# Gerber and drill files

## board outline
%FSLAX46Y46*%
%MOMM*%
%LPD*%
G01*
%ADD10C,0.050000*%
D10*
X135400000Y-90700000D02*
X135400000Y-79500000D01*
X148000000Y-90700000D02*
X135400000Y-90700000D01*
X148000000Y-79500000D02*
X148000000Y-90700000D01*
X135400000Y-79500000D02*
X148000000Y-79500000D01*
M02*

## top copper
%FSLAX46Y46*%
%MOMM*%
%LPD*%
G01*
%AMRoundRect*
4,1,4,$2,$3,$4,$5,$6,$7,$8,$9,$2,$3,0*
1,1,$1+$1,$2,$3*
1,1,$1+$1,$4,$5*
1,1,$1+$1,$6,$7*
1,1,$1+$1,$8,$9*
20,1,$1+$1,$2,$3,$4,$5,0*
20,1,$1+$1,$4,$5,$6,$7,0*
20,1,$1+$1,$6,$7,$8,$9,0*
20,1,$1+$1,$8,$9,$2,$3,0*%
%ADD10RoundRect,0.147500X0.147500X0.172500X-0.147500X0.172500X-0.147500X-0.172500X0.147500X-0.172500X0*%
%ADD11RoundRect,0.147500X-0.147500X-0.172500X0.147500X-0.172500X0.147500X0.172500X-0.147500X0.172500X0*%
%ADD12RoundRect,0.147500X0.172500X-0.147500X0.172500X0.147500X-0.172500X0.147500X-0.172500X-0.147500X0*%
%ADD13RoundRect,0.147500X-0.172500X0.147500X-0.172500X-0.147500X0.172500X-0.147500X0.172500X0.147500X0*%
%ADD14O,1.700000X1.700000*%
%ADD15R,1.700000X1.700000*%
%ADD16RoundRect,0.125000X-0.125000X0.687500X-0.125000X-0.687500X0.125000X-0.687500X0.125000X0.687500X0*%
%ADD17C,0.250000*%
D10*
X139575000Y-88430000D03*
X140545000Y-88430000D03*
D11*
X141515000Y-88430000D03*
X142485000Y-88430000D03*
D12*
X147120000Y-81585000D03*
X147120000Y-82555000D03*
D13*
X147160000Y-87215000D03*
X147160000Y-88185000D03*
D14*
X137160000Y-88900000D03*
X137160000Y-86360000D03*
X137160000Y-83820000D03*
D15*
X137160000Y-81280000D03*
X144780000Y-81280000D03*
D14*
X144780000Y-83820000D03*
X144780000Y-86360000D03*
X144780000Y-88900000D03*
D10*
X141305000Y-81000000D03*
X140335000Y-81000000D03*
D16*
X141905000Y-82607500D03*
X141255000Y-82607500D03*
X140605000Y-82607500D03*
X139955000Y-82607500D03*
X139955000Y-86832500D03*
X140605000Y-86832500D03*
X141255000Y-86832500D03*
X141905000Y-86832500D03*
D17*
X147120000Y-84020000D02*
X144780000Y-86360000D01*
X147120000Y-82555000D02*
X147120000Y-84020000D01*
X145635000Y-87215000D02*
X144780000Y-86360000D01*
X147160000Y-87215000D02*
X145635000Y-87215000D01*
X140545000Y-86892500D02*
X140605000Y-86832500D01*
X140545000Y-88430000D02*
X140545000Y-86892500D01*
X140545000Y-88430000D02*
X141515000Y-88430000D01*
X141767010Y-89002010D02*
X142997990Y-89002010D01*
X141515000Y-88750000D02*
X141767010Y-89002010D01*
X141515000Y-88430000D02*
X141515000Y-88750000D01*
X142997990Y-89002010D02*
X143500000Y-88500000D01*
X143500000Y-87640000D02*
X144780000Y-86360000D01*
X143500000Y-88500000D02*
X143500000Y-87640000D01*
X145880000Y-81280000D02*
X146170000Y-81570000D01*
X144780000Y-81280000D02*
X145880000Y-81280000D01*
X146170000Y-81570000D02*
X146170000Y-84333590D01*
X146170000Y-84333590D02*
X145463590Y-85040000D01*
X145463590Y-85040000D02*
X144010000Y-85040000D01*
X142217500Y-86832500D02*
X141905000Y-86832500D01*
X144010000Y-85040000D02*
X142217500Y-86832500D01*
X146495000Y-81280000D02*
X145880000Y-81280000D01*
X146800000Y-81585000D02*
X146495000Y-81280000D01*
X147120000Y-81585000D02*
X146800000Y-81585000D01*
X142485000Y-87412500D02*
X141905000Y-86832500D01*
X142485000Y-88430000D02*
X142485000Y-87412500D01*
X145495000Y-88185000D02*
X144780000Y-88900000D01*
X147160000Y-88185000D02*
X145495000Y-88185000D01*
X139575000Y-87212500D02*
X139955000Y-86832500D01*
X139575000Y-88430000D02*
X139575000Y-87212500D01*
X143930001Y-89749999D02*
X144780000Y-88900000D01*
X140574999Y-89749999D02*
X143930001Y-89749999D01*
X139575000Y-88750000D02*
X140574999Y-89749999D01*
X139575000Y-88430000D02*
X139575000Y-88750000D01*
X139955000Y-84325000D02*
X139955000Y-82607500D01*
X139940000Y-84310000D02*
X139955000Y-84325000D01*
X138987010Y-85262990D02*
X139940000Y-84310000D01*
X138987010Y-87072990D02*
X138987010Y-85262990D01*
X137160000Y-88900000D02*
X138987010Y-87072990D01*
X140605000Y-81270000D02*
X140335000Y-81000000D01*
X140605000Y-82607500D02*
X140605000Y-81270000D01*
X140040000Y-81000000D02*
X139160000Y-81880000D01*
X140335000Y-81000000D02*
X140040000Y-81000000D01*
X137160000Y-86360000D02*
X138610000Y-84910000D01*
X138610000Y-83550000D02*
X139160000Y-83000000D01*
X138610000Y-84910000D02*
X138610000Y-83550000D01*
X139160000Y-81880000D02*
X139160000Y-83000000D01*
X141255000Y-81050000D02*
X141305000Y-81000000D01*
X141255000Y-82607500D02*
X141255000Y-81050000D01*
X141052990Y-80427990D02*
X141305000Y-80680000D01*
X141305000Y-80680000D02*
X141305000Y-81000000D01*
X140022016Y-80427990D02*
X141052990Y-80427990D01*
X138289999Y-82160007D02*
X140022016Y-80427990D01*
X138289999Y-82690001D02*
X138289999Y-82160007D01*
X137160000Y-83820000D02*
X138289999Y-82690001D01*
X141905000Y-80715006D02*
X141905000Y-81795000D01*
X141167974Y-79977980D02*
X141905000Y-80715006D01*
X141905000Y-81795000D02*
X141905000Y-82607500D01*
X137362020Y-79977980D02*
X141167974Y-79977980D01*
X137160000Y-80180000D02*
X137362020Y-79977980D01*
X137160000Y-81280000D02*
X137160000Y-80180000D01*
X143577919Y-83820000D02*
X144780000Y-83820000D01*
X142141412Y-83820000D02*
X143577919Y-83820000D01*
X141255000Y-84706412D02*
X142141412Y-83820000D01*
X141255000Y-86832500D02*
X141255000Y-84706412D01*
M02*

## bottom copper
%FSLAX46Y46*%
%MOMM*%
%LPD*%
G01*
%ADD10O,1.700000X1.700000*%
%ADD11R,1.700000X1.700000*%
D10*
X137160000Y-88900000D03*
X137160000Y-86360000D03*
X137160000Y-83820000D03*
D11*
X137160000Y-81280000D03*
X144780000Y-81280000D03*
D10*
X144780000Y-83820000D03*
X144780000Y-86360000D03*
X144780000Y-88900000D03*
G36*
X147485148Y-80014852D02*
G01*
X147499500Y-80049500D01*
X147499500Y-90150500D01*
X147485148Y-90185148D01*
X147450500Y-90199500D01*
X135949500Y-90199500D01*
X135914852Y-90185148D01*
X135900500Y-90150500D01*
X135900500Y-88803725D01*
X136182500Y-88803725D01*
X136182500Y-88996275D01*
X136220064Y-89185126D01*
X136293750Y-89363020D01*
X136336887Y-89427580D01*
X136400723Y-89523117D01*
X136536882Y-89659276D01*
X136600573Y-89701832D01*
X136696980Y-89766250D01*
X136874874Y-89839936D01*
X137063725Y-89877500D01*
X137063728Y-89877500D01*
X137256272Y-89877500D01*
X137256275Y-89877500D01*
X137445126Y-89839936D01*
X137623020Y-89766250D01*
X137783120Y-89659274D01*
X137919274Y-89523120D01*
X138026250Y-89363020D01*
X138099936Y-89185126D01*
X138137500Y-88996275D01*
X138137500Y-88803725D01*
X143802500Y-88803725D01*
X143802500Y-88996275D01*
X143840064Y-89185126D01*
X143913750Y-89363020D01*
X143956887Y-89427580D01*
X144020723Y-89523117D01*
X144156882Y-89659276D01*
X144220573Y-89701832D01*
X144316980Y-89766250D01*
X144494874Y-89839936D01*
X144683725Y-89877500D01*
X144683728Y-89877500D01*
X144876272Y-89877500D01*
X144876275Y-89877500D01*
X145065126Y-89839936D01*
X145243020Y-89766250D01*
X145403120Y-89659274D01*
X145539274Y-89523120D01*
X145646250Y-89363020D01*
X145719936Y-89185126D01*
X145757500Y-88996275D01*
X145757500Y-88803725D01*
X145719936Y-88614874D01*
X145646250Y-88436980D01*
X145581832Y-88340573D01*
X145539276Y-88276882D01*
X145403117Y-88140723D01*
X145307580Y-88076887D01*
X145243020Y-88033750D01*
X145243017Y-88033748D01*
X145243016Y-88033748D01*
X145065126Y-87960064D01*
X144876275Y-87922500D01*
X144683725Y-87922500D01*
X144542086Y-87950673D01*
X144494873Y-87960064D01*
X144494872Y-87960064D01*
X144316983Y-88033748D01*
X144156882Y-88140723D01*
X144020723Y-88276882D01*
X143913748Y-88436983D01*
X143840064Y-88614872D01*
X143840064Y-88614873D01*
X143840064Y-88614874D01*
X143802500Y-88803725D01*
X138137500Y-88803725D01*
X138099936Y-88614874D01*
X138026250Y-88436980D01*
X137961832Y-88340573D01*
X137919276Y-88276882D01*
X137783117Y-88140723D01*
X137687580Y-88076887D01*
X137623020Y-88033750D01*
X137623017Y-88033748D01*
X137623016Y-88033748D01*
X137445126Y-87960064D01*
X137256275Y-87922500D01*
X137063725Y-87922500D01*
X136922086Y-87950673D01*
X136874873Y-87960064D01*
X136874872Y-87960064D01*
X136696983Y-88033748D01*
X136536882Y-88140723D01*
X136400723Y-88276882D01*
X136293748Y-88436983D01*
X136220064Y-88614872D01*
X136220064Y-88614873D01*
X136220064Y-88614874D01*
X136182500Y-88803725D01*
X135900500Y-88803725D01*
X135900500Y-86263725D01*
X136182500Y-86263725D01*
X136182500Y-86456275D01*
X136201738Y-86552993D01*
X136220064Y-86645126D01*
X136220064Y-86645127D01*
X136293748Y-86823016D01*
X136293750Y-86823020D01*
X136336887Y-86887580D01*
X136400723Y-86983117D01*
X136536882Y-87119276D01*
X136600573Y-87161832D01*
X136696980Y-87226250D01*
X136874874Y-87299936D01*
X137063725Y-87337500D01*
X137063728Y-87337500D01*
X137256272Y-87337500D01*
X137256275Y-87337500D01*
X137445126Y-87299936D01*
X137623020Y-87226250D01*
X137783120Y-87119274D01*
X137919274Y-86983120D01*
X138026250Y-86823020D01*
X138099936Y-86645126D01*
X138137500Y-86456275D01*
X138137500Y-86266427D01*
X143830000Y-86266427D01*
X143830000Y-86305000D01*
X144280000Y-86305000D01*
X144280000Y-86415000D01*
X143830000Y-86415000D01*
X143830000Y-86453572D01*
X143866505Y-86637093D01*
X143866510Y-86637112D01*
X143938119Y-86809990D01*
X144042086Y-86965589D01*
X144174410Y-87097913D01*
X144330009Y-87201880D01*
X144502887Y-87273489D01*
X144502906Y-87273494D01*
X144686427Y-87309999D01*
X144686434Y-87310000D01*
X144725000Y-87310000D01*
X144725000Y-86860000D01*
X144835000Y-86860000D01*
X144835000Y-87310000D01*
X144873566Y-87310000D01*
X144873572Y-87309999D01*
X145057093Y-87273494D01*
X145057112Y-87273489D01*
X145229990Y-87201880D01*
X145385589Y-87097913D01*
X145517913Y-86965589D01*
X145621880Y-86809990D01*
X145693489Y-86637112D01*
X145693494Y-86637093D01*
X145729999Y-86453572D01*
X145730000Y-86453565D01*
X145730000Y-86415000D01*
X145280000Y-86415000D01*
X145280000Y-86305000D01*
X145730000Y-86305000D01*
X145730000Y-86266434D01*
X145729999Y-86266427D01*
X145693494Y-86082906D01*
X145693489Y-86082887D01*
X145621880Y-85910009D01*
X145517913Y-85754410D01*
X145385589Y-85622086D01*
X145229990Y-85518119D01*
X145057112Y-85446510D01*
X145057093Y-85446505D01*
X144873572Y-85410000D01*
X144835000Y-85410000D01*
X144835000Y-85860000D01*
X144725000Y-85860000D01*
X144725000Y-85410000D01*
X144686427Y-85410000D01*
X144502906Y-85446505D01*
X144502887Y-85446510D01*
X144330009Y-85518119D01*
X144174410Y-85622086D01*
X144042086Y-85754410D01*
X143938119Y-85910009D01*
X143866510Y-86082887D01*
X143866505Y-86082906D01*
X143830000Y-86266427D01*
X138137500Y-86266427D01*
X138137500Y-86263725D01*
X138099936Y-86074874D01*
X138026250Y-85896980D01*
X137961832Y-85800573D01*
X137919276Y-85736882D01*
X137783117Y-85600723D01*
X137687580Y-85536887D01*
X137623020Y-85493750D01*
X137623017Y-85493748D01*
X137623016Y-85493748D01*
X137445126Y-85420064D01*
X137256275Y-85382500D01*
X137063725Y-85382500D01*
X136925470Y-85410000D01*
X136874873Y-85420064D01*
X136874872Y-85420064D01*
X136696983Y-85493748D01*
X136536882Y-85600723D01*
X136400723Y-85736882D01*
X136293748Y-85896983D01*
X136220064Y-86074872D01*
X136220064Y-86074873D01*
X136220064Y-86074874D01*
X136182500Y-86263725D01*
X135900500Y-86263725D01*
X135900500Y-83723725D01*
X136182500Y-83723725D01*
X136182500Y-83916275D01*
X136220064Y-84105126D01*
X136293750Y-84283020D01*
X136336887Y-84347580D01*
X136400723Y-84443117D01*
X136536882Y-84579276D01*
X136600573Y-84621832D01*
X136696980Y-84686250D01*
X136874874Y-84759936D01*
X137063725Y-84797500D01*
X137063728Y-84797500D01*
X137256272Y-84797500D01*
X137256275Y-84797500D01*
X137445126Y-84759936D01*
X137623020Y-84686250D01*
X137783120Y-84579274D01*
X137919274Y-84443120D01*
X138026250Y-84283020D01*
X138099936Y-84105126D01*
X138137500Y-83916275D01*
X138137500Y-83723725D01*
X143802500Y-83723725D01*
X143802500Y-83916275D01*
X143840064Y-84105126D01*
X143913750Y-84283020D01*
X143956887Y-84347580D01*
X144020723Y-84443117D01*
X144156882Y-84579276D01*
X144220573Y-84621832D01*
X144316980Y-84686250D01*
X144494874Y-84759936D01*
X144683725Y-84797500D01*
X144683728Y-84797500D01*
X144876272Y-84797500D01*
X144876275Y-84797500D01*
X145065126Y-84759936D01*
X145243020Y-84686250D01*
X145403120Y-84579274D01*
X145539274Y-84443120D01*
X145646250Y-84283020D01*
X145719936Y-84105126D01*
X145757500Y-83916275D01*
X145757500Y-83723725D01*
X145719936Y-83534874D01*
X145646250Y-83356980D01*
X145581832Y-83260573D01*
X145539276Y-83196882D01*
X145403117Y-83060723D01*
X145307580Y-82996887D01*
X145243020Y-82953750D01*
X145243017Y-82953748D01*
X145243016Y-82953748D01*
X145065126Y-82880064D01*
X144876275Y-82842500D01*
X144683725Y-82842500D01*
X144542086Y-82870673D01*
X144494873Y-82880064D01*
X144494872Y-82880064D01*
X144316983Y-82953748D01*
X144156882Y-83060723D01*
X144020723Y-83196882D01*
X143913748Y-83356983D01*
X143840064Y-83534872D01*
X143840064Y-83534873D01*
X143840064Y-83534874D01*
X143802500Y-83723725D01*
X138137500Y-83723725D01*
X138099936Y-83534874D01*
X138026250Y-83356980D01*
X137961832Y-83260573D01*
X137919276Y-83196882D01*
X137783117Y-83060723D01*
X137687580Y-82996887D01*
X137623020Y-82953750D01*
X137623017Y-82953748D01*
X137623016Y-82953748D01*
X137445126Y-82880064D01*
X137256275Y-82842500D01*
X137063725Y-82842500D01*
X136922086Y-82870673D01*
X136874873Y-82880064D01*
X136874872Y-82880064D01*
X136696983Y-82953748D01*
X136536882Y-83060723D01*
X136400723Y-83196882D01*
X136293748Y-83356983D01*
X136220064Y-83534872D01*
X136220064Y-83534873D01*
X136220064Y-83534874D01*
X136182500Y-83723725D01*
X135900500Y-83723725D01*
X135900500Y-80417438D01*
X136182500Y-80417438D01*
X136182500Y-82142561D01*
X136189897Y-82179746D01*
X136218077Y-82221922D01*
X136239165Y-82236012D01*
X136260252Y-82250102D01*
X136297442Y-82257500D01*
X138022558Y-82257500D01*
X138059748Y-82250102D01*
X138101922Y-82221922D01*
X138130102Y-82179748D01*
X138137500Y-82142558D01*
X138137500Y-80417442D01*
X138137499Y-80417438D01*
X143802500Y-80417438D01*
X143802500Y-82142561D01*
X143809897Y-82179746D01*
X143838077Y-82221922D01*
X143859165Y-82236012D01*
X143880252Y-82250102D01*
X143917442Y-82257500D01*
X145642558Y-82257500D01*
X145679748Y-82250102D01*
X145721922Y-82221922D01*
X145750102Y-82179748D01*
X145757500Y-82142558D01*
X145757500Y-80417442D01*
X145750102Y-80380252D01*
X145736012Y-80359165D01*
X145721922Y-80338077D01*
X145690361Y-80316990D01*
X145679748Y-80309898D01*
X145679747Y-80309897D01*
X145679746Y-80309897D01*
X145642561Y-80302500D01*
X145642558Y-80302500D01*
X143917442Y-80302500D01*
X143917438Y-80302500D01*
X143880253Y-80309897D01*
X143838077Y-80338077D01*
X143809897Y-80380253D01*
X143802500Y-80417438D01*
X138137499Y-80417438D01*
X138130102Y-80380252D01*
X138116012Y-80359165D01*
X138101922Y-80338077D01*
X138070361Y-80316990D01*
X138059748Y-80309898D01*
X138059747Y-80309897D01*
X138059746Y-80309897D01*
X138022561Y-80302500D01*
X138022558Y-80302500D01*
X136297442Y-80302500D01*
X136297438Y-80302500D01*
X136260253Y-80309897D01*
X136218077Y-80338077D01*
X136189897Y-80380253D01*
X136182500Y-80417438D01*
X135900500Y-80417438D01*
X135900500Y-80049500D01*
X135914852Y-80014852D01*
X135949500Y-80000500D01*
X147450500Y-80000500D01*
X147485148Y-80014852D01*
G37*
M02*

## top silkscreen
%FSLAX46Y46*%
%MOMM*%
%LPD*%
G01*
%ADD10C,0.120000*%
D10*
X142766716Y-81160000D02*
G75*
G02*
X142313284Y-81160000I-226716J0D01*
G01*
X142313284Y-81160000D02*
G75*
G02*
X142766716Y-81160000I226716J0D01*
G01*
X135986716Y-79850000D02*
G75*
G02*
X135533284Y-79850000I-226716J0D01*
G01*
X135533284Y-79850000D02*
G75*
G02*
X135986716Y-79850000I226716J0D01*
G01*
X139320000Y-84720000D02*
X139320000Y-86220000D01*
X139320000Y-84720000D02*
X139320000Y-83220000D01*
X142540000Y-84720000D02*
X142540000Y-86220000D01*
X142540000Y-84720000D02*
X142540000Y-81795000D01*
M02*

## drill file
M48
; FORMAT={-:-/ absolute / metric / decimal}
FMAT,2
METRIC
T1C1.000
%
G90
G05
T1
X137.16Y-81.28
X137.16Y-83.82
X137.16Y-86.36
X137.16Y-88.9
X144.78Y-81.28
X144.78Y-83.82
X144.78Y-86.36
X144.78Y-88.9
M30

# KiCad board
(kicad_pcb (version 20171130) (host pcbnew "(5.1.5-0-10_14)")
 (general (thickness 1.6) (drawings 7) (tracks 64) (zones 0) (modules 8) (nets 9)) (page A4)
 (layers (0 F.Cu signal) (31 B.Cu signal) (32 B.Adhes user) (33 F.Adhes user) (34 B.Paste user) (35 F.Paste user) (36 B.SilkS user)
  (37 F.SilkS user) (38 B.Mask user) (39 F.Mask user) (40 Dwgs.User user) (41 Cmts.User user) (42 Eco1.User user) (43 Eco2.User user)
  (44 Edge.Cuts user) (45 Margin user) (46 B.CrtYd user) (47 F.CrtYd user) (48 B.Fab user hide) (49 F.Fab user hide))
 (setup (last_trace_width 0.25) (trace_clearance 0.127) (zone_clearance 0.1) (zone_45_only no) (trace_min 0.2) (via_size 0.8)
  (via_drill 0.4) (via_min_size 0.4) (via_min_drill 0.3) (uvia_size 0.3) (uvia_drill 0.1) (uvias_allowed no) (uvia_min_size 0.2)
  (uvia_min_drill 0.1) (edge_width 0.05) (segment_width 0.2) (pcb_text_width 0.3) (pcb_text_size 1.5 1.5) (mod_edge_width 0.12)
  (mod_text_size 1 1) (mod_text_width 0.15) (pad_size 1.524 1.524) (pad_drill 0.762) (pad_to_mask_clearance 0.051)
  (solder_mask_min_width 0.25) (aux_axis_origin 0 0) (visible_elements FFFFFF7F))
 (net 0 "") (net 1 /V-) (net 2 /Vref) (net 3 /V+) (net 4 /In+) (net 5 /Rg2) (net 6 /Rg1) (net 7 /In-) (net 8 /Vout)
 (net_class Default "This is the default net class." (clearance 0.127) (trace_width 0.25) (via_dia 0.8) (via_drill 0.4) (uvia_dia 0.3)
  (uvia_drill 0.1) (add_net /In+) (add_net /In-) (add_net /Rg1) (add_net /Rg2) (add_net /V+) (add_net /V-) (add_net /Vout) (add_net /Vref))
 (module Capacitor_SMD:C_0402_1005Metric (layer F.Cu) (at 140.06 88.43 180)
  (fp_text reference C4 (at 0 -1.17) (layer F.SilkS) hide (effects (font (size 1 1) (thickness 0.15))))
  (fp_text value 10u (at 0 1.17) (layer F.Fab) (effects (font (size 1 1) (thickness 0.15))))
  (pad 2 smd roundrect (at 0.485 0 180) (size 0.59 0.64) (layers F.Cu F.Paste F.Mask) (roundrect_rratio 0.25) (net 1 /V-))
  (pad 1 smd roundrect (at -0.485 0 180) (size 0.59 0.64) (layers F.Cu F.Paste F.Mask) (roundrect_rratio 0.25) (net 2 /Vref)))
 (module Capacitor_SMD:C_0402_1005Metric (layer F.Cu) (at 142 88.43)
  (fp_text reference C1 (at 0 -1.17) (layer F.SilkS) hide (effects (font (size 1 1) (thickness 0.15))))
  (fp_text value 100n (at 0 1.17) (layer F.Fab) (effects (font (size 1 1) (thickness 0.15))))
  (pad 1 smd roundrect (at -0.485 0) (size 0.59 0.64) (layers F.Cu F.Paste F.Mask) (roundrect_rratio 0.25) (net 2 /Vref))
  (pad 2 smd roundrect (at 0.485 0) (size 0.59 0.64) (layers F.Cu F.Paste F.Mask) (roundrect_rratio 0.25) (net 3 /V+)))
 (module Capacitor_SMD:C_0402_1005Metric (layer F.Cu) (at 147.12 82.07 90)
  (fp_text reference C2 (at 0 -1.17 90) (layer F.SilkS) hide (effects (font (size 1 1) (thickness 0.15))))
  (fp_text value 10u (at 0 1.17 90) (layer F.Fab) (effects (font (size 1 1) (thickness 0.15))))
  (pad 2 smd roundrect (at 0.485 0 90) (size 0.59 0.64) (layers F.Cu F.Paste F.Mask) (roundrect_rratio 0.25) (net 3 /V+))
  (pad 1 smd roundrect (at -0.485 0 90) (size 0.59 0.64) (layers F.Cu F.Paste F.Mask) (roundrect_rratio 0.25) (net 2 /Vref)))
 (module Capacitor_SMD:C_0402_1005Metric (layer F.Cu) (at 147.16 87.7 270)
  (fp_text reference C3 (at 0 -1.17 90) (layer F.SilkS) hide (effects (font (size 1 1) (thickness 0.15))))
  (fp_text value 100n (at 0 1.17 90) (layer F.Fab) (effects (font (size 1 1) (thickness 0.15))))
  (pad 1 smd roundrect (at -0.485 0 270) (size 0.59 0.64) (layers F.Cu F.Paste F.Mask) (roundrect_rratio 0.25) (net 2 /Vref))
  (pad 2 smd roundrect (at 0.485 0 270) (size 0.59 0.64) (layers F.Cu F.Paste F.Mask) (roundrect_rratio 0.25) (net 1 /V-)))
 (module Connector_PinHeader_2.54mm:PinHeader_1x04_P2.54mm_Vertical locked (layer B.Cu) (at 137.16 81.28 180)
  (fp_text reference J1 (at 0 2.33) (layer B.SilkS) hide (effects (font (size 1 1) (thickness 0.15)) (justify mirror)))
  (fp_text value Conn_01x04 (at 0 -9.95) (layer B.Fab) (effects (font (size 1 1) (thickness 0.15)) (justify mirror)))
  (pad 4 thru_hole oval (at 0 -7.62 180) (size 1.7 1.7) (drill 1) (layers *.Cu *.Mask) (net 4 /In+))
  (pad 3 thru_hole oval (at 0 -5.08 180) (size 1.7 1.7) (drill 1) (layers *.Cu *.Mask) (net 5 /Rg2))
  (pad 2 thru_hole oval (at 0 -2.54 180) (size 1.7 1.7) (drill 1) (layers *.Cu *.Mask) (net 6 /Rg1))
  (pad 1 thru_hole rect (at 0 0 180) (size 1.7 1.7) (drill 1) (layers *.Cu *.Mask) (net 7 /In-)))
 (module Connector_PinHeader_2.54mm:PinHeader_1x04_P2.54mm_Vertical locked (layer B.Cu) (at 144.78 81.28 180)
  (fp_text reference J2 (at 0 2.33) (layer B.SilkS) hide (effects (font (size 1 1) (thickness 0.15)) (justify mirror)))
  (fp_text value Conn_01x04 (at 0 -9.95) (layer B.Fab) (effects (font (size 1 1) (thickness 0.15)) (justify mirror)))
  (pad 1 thru_hole rect (at 0 0 180) (size 1.7 1.7) (drill 1) (layers *.Cu *.Mask) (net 3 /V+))
  (pad 2 thru_hole oval (at 0 -2.54 180) (size 1.7 1.7) (drill 1) (layers *.Cu *.Mask) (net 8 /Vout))
  (pad 3 thru_hole oval (at 0 -5.08 180) (size 1.7 1.7) (drill 1) (layers *.Cu *.Mask) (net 2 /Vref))
  (pad 4 thru_hole oval (at 0 -7.62 180) (size 1.7 1.7) (drill 1) (layers *.Cu *.Mask) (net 1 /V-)))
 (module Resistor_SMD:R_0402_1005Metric (layer F.Cu) (at 140.82 81 180)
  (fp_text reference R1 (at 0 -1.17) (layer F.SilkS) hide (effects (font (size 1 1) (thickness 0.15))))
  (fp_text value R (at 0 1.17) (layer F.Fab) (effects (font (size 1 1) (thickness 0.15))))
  (pad 1 smd roundrect (at -0.485 0 180) (size 0.59 0.64) (layers F.Cu F.Paste F.Mask) (roundrect_rratio 0.25) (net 6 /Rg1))
  (pad 2 smd roundrect (at 0.485 0 180) (size 0.59 0.64) (layers F.Cu F.Paste F.Mask) (roundrect_rratio 0.25) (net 5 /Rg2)))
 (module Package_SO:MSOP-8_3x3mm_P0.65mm (layer F.Cu) (at 140.93 84.72 270)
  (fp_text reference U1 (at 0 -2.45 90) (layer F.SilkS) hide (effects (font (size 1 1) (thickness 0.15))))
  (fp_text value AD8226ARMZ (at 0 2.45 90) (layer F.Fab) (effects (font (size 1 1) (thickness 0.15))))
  (fp_line (start 0 1.61) (end 1.5 1.61) (layer F.SilkS) (width 0.12))
  (fp_line (start 0 1.61) (end -1.5 1.61) (layer F.SilkS) (width 0.12))
  (fp_line (start 0 -1.61) (end 1.5 -1.61) (layer F.SilkS) (width 0.12))
  (fp_line (start 0 -1.61) (end -2.925 -1.61) (layer F.SilkS) (width 0.12))
  (pad 1 smd roundrect (at -2.1125 -0.975 270) (size 1.625 0.5) (layers F.Cu F.Paste F.Mask) (roundrect_rratio 0.25) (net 7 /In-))
  (pad 2 smd roundrect (at -2.1125 -0.325 270) (size 1.625 0.5) (layers F.Cu F.Paste F.Mask) (roundrect_rratio 0.25) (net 6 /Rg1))
  (pad 3 smd roundrect (at -2.1125 0.325 270) (size 1.625 0.5) (layers F.Cu F.Paste F.Mask) (roundrect_rratio 0.25) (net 5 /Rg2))
  (pad 4 smd roundrect (at -2.1125 0.975 270) (size 1.625 0.5) (layers F.Cu F.Paste F.Mask) (roundrect_rratio 0.25) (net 4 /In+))
  (pad 5 smd roundrect (at 2.1125 0.975 270) (size 1.625 0.5) (layers F.Cu F.Paste F.Mask) (roundrect_rratio 0.25) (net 1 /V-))
  (pad 6 smd roundrect (at 2.1125 0.325 270) (size 1.625 0.5) (layers F.Cu F.Paste F.Mask) (roundrect_rratio 0.25) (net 2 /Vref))
  (pad 7 smd roundrect (at 2.1125 -0.325 270) (size 1.625 0.5) (layers F.Cu F.Paste F.Mask) (roundrect_rratio 0.25) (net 8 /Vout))
  (pad 8 smd roundrect (at 2.1125 -0.975 270) (size 1.625 0.5) (layers F.Cu F.Paste F.Mask) (roundrect_rratio 0.25) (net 3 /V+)))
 (gr_circle (center 142.54 81.16) (end 142.69 81.33) (layer F.SilkS) (width 0.12))
 (gr_circle (center 135.76 79.85) (end 135.91 80.02) (layer F.SilkS) (width 0.12))
 (gr_line (start 135.4 90.7) (end 135.4 79.5) (layer Edge.Cuts) (width 0.05))
 (gr_line (start 148 90.7) (end 135.4 90.7) (layer Edge.Cuts) (width 0.05))
 (gr_line (start 148 79.5) (end 148 90.7) (layer Edge.Cuts) (width 0.05))
 (gr_line (start 135.4 79.5) (end 148 79.5) (layer Edge.Cuts) (width 0.05))
 (segment (start 147.12 84.02) (end 144.78 86.36) (width 0.25) (layer F.Cu) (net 2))
 (segment (start 147.12 82.555) (end 147.12 84.02) (width 0.25) (layer F.Cu) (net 2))
 (segment (start 145.635 87.215) (end 144.78 86.36) (width 0.25) (layer F.Cu) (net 2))
 (segment (start 147.16 87.215) (end 145.635 87.215) (width 0.25) (layer F.Cu) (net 2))
 (segment (start 140.545 86.8925) (end 140.605 86.8325) (width 0.25) (layer F.Cu) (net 2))
 (segment (start 140.545 88.43) (end 140.545 86.8925) (width 0.25) (layer F.Cu) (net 2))
 (segment (start 140.545 88.43) (end 141.515 88.43) (width 0.25) (layer F.Cu) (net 2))
 (segment (start 141.76701 89.00201) (end 142.99799 89.00201) (width 0.25) (layer F.Cu) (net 2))
 (segment (start 141.515 88.75) (end 141.76701 89.00201) (width 0.25) (layer F.Cu) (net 2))
 (segment (start 141.515 88.43) (end 141.515 88.75) (width 0.25) (layer F.Cu) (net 2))
 (segment (start 142.99799 89.00201) (end 143.5 88.5) (width 0.25) (layer F.Cu) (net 2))
 (segment (start 143.5 87.64) (end 144.78 86.36) (width 0.25) (layer F.Cu) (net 2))
 (segment (start 143.5 88.5) (end 143.5 87.64) (width 0.25) (layer F.Cu) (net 2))
 (segment (start 145.88 81.28) (end 146.17 81.57) (width 0.25) (layer F.Cu) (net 3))
 (segment (start 144.78 81.28) (end 145.88 81.28) (width 0.25) (layer F.Cu) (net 3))
 (segment (start 146.17 81.57) (end 146.17 84.33359) (width 0.25) (layer F.Cu) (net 3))
 (segment (start 146.17 84.33359) (end 145.46359 85.04) (width 0.25) (layer F.Cu) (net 3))
 (segment (start 145.46359 85.04) (end 144.01 85.04) (width 0.25) (layer F.Cu) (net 3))
 (segment (start 142.2175 86.8325) (end 141.905 86.8325) (width 0.25) (layer F.Cu) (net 3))
 (segment (start 144.01 85.04) (end 142.2175 86.8325) (width 0.25) (layer F.Cu) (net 3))
 (segment (start 146.495 81.28) (end 145.88 81.28) (width 0.25) (layer F.Cu) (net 3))
 (segment (start 146.8 81.585) (end 146.495 81.28) (width 0.25) (layer F.Cu) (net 3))
 (segment (start 147.12 81.585) (end 146.8 81.585) (width 0.25) (layer F.Cu) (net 3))
 (segment (start 142.485 87.4125) (end 141.905 86.8325) (width 0.25) (layer F.Cu) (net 3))
 (segment (start 142.485 88.43) (end 142.485 87.4125) (width 0.25) (layer F.Cu) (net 3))
 (segment (start 145.495 88.185) (end 144.78 88.9) (width 0.25) (layer F.Cu) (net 1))
 (segment (start 147.16 88.185) (end 145.495 88.185) (width 0.25) (layer F.Cu) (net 1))
 (segment (start 139.575 87.2125) (end 139.955 86.8325) (width 0.25) (layer F.Cu) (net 1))
 (segment (start 139.575 88.43) (end 139.575 87.2125) (width 0.25) (layer F.Cu) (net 1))
 (segment (start 143.930001 89.749999) (end 144.78 88.9) (width 0.25) (layer F.Cu) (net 1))
 (segment (start 140.574999 89.749999) (end 143.930001 89.749999) (width 0.25) (layer F.Cu) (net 1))
 (segment (start 139.575 88.75) (end 140.574999 89.749999) (width 0.25) (layer F.Cu) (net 1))
 (segment (start 139.575 88.43) (end 139.575 88.75) (width 0.25) (layer F.Cu) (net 1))
 (segment (start 139.955 84.325) (end 139.955 82.6075) (width 0.25) (layer F.Cu) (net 4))
 (segment (start 139.94 84.31) (end 139.955 84.325) (width 0.25) (layer F.Cu) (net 4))
 (segment (start 138.98701 85.26299) (end 139.94 84.31) (width 0.25) (layer F.Cu) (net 4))
 (segment (start 138.98701 87.07299) (end 138.98701 85.26299) (width 0.25) (layer F.Cu) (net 4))
 (segment (start 137.16 88.9) (end 138.98701 87.07299) (width 0.25) (layer F.Cu) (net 4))
 (segment (start 140.605 81.27) (end 140.335 81) (width 0.25) (layer F.Cu) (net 5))
 (segment (start 140.605 82.6075) (end 140.605 81.27) (width 0.25) (layer F.Cu) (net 5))
 (segment (start 140.04 81) (end 139.16 81.88) (width 0.25) (layer F.Cu) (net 5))
 (segment (start 140.335 81) (end 140.04 81) (width 0.25) (layer F.Cu) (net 5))
 (segment (start 137.16 86.36) (end 138.61 84.91) (width 0.25) (layer F.Cu) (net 5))
 (segment (start 138.61 83.55) (end 139.16 83) (width 0.25) (layer F.Cu) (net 5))
 (segment (start 138.61 84.91) (end 138.61 83.55) (width 0.25) (layer F.Cu) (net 5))
 (segment (start 139.16 81.88) (end 139.16 83) (width 0.25) (layer F.Cu) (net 5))
 (segment (start 141.255 81.05) (end 141.305 81) (width 0.25) (layer F.Cu) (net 6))
 (segment (start 141.255 82.6075) (end 141.255 81.05) (width 0.25) (layer F.Cu) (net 6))
 (segment (start 141.05299 80.42799) (end 141.305 80.68) (width 0.25) (layer F.Cu) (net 6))
 (segment (start 141.305 80.68) (end 141.305 81) (width 0.25) (layer F.Cu) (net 6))
 (segment (start 140.022016 80.42799) (end 141.05299 80.42799) (width 0.25) (layer F.Cu) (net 6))
 (segment (start 138.289999 82.160007) (end 140.022016 80.42799) (width 0.25) (layer F.Cu) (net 6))
 (segment (start 138.289999 82.690001) (end 138.289999 82.160007) (width 0.25) (layer F.Cu) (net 6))
 (segment (start 137.16 83.82) (end 138.289999 82.690001) (width 0.25) (layer F.Cu) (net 6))
 (segment (start 141.905 80.715006) (end 141.905 81.795) (width 0.25) (layer F.Cu) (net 7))
 (segment (start 141.167974 79.97798) (end 141.905 80.715006) (width 0.25) (layer F.Cu) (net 7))
 (segment (start 141.905 81.795) (end 141.905 82.6075) (width 0.25) (layer F.Cu) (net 7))
 (segment (start 137.36202 79.97798) (end 141.167974 79.97798) (width 0.25) (layer F.Cu) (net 7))
 (segment (start 137.16 80.18) (end 137.36202 79.97798) (width 0.25) (layer F.Cu) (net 7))
 (segment (start 137.16 81.28) (end 137.16 80.18) (width 0.25) (layer F.Cu) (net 7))
 (segment (start 143.577919 83.82) (end 144.78 83.82) (width 0.25) (layer F.Cu) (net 8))
 (segment (start 142.141412 83.82) (end 143.577919 83.82) (width 0.25) (layer F.Cu) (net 8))
 (segment (start 141.255 84.706412) (end 142.141412 83.82) (width 0.25) (layer F.Cu) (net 8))
 (segment (start 141.255 86.8325) (end 141.255 84.706412) (width 0.25) (layer F.Cu) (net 8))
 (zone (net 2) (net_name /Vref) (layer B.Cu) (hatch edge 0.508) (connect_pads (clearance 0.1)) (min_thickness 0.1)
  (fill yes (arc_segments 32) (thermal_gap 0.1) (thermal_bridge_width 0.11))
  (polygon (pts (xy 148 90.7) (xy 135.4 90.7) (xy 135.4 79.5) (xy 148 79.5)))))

